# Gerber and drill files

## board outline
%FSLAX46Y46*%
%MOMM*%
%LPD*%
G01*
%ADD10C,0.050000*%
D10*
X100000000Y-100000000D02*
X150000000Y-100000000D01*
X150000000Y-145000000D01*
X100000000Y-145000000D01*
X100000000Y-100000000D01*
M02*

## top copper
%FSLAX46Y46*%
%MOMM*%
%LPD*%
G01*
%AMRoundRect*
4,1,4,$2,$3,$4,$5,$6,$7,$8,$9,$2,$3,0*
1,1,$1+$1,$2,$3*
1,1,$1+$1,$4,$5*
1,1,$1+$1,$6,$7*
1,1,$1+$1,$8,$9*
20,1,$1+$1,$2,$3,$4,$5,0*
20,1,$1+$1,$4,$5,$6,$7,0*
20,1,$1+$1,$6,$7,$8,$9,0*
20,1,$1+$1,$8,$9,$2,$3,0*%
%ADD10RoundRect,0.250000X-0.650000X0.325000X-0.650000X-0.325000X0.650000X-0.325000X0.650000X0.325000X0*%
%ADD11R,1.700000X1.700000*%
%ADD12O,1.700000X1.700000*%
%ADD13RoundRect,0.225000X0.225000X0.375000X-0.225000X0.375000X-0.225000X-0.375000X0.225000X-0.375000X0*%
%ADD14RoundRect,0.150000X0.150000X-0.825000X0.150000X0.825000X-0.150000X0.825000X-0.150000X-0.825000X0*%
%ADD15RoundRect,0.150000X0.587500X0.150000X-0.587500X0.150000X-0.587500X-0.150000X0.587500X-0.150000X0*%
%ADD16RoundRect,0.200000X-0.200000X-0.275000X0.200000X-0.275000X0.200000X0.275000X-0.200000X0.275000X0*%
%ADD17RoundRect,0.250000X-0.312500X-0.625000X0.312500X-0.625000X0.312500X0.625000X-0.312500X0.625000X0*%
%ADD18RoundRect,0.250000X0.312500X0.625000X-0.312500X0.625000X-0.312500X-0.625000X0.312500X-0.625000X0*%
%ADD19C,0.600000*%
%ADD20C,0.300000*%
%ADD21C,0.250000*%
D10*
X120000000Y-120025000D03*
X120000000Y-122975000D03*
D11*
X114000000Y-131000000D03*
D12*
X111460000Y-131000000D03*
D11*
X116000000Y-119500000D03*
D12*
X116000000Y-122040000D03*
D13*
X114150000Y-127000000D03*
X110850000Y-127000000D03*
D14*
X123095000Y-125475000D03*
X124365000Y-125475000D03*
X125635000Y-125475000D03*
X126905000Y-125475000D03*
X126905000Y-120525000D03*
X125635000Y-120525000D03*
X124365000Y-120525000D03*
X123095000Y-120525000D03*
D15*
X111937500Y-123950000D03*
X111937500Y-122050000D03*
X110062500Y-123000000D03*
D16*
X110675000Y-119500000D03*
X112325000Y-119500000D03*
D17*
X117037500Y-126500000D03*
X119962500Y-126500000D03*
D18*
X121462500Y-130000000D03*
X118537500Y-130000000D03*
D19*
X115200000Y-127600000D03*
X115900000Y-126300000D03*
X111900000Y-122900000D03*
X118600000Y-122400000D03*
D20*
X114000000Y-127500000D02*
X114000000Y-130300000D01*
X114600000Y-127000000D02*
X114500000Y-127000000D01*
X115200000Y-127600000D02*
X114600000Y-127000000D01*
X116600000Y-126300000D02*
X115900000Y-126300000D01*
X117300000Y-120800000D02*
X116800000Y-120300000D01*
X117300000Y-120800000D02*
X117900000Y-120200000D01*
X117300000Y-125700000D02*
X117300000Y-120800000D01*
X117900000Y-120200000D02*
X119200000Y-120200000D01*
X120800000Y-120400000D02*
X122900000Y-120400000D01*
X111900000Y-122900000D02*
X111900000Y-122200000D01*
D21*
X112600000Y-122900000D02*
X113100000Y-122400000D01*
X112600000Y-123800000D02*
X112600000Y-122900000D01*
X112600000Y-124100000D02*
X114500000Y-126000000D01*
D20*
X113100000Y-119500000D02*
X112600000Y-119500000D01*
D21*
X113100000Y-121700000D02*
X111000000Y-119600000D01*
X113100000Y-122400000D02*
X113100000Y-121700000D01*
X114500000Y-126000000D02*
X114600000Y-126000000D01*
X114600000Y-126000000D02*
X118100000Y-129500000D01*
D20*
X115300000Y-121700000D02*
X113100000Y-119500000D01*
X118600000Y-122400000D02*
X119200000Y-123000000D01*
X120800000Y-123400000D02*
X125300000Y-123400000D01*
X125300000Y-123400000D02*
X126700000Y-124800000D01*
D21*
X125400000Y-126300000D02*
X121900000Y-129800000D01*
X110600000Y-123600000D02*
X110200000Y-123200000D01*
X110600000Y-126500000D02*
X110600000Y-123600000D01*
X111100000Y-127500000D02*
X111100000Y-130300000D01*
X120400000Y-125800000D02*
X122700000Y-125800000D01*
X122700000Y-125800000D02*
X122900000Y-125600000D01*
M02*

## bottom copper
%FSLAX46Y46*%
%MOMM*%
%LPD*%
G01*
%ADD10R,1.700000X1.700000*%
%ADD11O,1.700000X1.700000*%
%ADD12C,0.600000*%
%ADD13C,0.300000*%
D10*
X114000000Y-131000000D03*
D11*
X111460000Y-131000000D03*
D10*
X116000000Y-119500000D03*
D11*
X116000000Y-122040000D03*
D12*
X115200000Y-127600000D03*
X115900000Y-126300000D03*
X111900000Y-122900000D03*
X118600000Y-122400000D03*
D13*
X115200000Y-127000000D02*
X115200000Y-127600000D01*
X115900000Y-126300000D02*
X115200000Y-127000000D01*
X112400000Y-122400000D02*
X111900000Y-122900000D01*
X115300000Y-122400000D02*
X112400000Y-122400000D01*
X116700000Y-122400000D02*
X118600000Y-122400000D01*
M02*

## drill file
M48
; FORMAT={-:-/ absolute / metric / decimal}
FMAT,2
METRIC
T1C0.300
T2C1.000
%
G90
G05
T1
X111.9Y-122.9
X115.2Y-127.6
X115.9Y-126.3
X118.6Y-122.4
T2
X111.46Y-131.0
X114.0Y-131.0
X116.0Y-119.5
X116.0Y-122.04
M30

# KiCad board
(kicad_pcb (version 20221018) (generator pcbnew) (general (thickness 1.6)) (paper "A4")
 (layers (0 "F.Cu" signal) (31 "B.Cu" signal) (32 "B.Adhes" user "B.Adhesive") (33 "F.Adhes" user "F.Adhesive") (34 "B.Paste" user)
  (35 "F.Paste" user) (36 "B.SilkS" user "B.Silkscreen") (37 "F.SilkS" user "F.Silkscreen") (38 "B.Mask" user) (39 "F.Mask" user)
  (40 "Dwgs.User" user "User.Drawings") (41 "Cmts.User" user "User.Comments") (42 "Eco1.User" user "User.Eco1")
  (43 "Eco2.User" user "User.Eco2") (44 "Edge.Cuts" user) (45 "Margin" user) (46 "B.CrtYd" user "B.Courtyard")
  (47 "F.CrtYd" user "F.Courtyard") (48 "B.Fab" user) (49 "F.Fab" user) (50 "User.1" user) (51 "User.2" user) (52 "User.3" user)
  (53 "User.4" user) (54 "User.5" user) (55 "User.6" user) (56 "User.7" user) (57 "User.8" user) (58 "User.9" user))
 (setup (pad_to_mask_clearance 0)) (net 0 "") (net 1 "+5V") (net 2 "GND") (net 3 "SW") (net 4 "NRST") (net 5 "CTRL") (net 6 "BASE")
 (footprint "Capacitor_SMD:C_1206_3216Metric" (layer "F.Cu") (at 120 121.5 -90)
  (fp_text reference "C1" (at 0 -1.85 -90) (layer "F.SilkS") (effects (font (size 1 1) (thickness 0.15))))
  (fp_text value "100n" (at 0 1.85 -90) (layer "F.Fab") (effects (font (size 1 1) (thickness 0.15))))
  (pad "1" smd roundrect (at -1.475 0 270) (size 1.15 1.8) (layers "F.Cu" "F.Paste" "F.Mask") (roundrect_rratio 0.217391) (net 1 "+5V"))
  (pad "2" smd roundrect (at 1.475 0 270) (size 1.15 1.8) (layers "F.Cu" "F.Paste" "F.Mask") (roundrect_rratio 0.217391) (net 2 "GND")))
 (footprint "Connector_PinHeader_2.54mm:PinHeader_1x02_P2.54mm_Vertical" (layer "F.Cu") (at 114 131 -90)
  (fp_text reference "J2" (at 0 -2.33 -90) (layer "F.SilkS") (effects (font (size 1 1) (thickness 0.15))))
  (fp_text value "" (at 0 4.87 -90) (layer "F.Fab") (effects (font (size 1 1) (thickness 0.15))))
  (pad "1" thru_hole rect (at 0 0 270) (size 1.7 1.7) (drill 1) (layers "*.Cu" "*.Mask") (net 1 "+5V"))
  (pad "2" thru_hole oval (at 0 2.54 270) (size 1.7 1.7) (drill 1) (layers "*.Cu" "*.Mask") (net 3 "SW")))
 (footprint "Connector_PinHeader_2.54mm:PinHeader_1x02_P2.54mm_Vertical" (layer "F.Cu") (at 116 119.5)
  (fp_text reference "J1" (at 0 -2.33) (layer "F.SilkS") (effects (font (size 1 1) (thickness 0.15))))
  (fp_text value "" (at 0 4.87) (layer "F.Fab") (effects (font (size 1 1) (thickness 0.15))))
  (pad "1" thru_hole rect (at 0 0) (size 1.7 1.7) (drill 1) (layers "*.Cu" "*.Mask") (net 1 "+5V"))
  (pad "2" thru_hole oval (at 0 2.54) (size 1.7 1.7) (drill 1) (layers "*.Cu" "*.Mask") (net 2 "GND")))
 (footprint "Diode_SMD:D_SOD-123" (layer "F.Cu") (at 112.5 127 180)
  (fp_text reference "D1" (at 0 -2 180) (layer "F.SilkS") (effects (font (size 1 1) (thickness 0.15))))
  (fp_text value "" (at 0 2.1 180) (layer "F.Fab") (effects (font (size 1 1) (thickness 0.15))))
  (pad "1" smd roundrect (at -1.65 0 180) (size 0.9 1.2) (layers "F.Cu" "F.Paste" "F.Mask") (roundrect_rratio 0.25) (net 1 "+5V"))
  (pad "2" smd roundrect (at 1.65 0 180) (size 0.9 1.2) (layers "F.Cu" "F.Paste" "F.Mask") (roundrect_rratio 0.25) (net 3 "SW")))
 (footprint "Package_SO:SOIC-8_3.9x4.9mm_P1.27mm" (layer "F.Cu") (at 125 123 90)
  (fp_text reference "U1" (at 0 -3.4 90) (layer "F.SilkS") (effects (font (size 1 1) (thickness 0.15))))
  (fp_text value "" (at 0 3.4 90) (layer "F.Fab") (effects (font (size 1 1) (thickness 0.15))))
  (pad "1" smd roundrect (at -2.475 -1.905 90) (size 1.95 0.6) (layers "F.Cu" "F.Paste" "F.Mask") (roundrect_rratio 0.25) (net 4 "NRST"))
  (pad "2" smd roundrect (at -2.475 -0.635 90) (size 1.95 0.6) (layers "F.Cu" "F.Paste" "F.Mask") (roundrect_rratio 0.25))
  (pad "3" smd roundrect (at -2.475 0.635 90) (size 1.95 0.6) (layers "F.Cu" "F.Paste" "F.Mask") (roundrect_rratio 0.25) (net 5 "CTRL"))
  (pad "4" smd roundrect (at -2.475 1.905 90) (size 1.95 0.6) (layers "F.Cu" "F.Paste" "F.Mask") (roundrect_rratio 0.25) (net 2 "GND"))
  (pad "5" smd roundrect (at 2.475 1.905 90) (size 1.95 0.6) (layers "F.Cu" "F.Paste" "F.Mask") (roundrect_rratio 0.25))
  (pad "6" smd roundrect (at 2.475 0.635 90) (size 1.95 0.6) (layers "F.Cu" "F.Paste" "F.Mask") (roundrect_rratio 0.25))
  (pad "7" smd roundrect (at 2.475 -0.635 90) (size 1.95 0.6) (layers "F.Cu" "F.Paste" "F.Mask") (roundrect_rratio 0.25))
  (pad "8" smd roundrect (at 2.475 -1.905 90) (size 1.95 0.6) (layers "F.Cu" "F.Paste" "F.Mask") (roundrect_rratio 0.25) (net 1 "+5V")))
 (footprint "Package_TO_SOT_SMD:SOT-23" (layer "F.Cu") (at 111 123 180)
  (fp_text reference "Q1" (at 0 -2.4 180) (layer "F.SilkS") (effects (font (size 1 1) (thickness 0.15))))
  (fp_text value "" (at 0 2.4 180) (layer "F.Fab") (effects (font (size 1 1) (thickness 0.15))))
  (pad "1" smd roundrect (at -0.9375 -0.95 180) (size 1.475 0.6) (layers "F.Cu" "F.Paste" "F.Mask") (roundrect_rratio 0.25) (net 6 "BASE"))
  (pad "2" smd roundrect (at -0.9375 0.95 180) (size 1.475 0.6) (layers "F.Cu" "F.Paste" "F.Mask") (roundrect_rratio 0.25) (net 2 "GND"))
  (pad "3" smd roundrect (at 0.9375 0 180) (size 1.475 0.6) (layers "F.Cu" "F.Paste" "F.Mask") (roundrect_rratio 0.25) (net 3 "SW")))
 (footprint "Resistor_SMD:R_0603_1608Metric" (layer "F.Cu") (at 111.5 119.5)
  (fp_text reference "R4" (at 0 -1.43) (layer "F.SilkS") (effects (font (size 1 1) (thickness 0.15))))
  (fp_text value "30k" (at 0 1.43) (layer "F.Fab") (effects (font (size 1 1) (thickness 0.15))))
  (pad "1" smd roundrect (at -0.825 0) (size 0.8 0.95) (layers "F.Cu" "F.Paste" "F.Mask") (roundrect_rratio 0.25) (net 6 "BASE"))
  (pad "2" smd roundrect (at 0.825 0) (size 0.8 0.95) (layers "F.Cu" "F.Paste" "F.Mask") (roundrect_rratio 0.25) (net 2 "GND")))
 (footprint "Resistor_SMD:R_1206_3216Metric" (layer "F.Cu") (at 118.5 126.5)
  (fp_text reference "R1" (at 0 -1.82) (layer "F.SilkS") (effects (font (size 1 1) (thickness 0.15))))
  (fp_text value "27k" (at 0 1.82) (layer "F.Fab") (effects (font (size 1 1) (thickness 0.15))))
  (pad "1" smd roundrect (at -1.4625 0) (size 1.125 1.75) (layers "F.Cu" "F.Paste" "F.Mask") (roundrect_rratio 0.222222) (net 1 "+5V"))
  (pad "2" smd roundrect (at 1.4625 0) (size 1.125 1.75) (layers "F.Cu" "F.Paste" "F.Mask") (roundrect_rratio 0.222222) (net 4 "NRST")))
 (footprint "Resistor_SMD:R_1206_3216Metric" (layer "F.Cu") (at 120 130 180)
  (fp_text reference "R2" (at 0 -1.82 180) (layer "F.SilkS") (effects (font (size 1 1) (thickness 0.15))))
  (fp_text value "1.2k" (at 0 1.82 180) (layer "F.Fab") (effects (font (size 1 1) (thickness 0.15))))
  (pad "1" smd roundrect (at -1.4625 0 180) (size 1.125 1.75) (layers "F.Cu" "F.Paste" "F.Mask") (roundrect_rratio 0.222222) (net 5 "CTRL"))
  (pad "2" smd roundrect (at 1.4625 0 180) (size 1.125 1.75) (layers "F.Cu" "F.Paste" "F.Mask") (roundrect_rratio 0.222222) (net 6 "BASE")))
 (gr_rect (start 100 100) (end 150 145) (stroke (width 0.05) (type default)) (fill none) (layer "Edge.Cuts"))
 (segment (start 114 127.5) (end 114 130.3) (width 0.3) (layer "F.Cu") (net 1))
 (segment (start 114.6 127) (end 114.5 127) (width 0.3) (layer "F.Cu") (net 1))
 (segment (start 115.2 127.6) (end 114.6 127) (width 0.3) (layer "F.Cu") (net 1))
 (segment (start 116.6 126.3) (end 115.9 126.3) (width 0.3) (layer "F.Cu") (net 1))
 (segment (start 117.3 120.8) (end 116.8 120.3) (width 0.3) (layer "F.Cu") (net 1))
 (segment (start 117.3 120.8) (end 117.9 120.2) (width 0.3) (layer "F.Cu") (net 1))
 (segment (start 117.3 125.7) (end 117.3 120.8) (width 0.3) (layer "F.Cu") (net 1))
 (segment (start 117.9 120.2) (end 119.2 120.2) (width 0.3) (layer "F.Cu") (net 1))
 (segment (start 120.8 120.4) (end 122.9 120.4) (width 0.3) (layer "F.Cu") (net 1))
 (via (at 115.2 127.6) (size 0.6) (drill 0.3) (layers "F.Cu" "B.Cu") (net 1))
 (via (at 115.9 126.3) (size 0.6) (drill 0.3) (layers "F.Cu" "B.Cu") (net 1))
 (segment (start 111.9 122.9) (end 111.9 122.2) (width 0.3) (layer "F.Cu") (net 2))
 (segment (start 112.6 122.9) (end 113.1 122.4) (width 0.25) (layer "F.Cu") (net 6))
 (segment (start 112.6 123.8) (end 112.6 122.9) (width 0.25) (layer "F.Cu") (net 6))
 (segment (start 112.6 124.1) (end 114.5 126) (width 0.25) (layer "F.Cu") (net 6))
 (segment (start 113.1 119.5) (end 112.6 119.5) (width 0.3) (layer "F.Cu") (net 2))
 (segment (start 113.1 121.7) (end 111 119.6) (width 0.25) (layer "F.Cu") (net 6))
 (segment (start 113.1 122.4) (end 113.1 121.7) (width 0.25) (layer "F.Cu") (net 6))
 (segment (start 114.5 126) (end 114.6 126) (width 0.25) (layer "F.Cu") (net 6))
 (segment (start 114.6 126) (end 118.1 129.5) (width 0.25) (layer "F.Cu") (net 6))
 (segment (start 115.2 127) (end 115.2 127.6) (width 0.3) (layer "B.Cu") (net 1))
 (segment (start 115.3 121.7) (end 113.1 119.5) (width 0.3) (layer "F.Cu") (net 2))
 (segment (start 115.9 126.3) (end 115.2 127) (width 0.3) (layer "B.Cu") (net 1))
 (segment (start 118.6 122.4) (end 119.2 123) (width 0.3) (layer "F.Cu") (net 2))
 (segment (start 120.8 123.4) (end 125.3 123.4) (width 0.3) (layer "F.Cu") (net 2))
 (segment (start 125.3 123.4) (end 126.7 124.8) (width 0.3) (layer "F.Cu") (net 2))
 (segment (start 125.4 126.3) (end 121.9 129.8) (width 0.25) (layer "F.Cu") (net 5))
 (via (at 111.9 122.9) (size 0.6) (drill 0.3) (layers "F.Cu" "B.Cu") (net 2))
 (via (at 118.6 122.4) (size 0.6) (drill 0.3) (layers "F.Cu" "B.Cu") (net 2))
 (segment (start 110.6 123.6) (end 110.2 123.2) (width 0.25) (layer "F.Cu") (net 3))
 (segment (start 110.6 126.5) (end 110.6 123.6) (width 0.25) (layer "F.Cu") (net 3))
 (segment (start 111.1 127.5) (end 111.1 130.3) (width 0.25) (layer "F.Cu") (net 3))
 (segment (start 112.4 122.4) (end 111.9 122.9) (width 0.3) (layer "B.Cu") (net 2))
 (segment (start 115.3 122.4) (end 112.4 122.4) (width 0.3) (layer "B.Cu") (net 2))
 (segment (start 116.7 122.4) (end 118.6 122.4) (width 0.3) (layer "B.Cu") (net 2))
 (segment (start 120.4 125.8) (end 122.7 125.8) (width 0.25) (layer "F.Cu") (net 4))
 (segment (start 122.7 125.8) (end 122.9 125.6) (width 0.25) (layer "F.Cu") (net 4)))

